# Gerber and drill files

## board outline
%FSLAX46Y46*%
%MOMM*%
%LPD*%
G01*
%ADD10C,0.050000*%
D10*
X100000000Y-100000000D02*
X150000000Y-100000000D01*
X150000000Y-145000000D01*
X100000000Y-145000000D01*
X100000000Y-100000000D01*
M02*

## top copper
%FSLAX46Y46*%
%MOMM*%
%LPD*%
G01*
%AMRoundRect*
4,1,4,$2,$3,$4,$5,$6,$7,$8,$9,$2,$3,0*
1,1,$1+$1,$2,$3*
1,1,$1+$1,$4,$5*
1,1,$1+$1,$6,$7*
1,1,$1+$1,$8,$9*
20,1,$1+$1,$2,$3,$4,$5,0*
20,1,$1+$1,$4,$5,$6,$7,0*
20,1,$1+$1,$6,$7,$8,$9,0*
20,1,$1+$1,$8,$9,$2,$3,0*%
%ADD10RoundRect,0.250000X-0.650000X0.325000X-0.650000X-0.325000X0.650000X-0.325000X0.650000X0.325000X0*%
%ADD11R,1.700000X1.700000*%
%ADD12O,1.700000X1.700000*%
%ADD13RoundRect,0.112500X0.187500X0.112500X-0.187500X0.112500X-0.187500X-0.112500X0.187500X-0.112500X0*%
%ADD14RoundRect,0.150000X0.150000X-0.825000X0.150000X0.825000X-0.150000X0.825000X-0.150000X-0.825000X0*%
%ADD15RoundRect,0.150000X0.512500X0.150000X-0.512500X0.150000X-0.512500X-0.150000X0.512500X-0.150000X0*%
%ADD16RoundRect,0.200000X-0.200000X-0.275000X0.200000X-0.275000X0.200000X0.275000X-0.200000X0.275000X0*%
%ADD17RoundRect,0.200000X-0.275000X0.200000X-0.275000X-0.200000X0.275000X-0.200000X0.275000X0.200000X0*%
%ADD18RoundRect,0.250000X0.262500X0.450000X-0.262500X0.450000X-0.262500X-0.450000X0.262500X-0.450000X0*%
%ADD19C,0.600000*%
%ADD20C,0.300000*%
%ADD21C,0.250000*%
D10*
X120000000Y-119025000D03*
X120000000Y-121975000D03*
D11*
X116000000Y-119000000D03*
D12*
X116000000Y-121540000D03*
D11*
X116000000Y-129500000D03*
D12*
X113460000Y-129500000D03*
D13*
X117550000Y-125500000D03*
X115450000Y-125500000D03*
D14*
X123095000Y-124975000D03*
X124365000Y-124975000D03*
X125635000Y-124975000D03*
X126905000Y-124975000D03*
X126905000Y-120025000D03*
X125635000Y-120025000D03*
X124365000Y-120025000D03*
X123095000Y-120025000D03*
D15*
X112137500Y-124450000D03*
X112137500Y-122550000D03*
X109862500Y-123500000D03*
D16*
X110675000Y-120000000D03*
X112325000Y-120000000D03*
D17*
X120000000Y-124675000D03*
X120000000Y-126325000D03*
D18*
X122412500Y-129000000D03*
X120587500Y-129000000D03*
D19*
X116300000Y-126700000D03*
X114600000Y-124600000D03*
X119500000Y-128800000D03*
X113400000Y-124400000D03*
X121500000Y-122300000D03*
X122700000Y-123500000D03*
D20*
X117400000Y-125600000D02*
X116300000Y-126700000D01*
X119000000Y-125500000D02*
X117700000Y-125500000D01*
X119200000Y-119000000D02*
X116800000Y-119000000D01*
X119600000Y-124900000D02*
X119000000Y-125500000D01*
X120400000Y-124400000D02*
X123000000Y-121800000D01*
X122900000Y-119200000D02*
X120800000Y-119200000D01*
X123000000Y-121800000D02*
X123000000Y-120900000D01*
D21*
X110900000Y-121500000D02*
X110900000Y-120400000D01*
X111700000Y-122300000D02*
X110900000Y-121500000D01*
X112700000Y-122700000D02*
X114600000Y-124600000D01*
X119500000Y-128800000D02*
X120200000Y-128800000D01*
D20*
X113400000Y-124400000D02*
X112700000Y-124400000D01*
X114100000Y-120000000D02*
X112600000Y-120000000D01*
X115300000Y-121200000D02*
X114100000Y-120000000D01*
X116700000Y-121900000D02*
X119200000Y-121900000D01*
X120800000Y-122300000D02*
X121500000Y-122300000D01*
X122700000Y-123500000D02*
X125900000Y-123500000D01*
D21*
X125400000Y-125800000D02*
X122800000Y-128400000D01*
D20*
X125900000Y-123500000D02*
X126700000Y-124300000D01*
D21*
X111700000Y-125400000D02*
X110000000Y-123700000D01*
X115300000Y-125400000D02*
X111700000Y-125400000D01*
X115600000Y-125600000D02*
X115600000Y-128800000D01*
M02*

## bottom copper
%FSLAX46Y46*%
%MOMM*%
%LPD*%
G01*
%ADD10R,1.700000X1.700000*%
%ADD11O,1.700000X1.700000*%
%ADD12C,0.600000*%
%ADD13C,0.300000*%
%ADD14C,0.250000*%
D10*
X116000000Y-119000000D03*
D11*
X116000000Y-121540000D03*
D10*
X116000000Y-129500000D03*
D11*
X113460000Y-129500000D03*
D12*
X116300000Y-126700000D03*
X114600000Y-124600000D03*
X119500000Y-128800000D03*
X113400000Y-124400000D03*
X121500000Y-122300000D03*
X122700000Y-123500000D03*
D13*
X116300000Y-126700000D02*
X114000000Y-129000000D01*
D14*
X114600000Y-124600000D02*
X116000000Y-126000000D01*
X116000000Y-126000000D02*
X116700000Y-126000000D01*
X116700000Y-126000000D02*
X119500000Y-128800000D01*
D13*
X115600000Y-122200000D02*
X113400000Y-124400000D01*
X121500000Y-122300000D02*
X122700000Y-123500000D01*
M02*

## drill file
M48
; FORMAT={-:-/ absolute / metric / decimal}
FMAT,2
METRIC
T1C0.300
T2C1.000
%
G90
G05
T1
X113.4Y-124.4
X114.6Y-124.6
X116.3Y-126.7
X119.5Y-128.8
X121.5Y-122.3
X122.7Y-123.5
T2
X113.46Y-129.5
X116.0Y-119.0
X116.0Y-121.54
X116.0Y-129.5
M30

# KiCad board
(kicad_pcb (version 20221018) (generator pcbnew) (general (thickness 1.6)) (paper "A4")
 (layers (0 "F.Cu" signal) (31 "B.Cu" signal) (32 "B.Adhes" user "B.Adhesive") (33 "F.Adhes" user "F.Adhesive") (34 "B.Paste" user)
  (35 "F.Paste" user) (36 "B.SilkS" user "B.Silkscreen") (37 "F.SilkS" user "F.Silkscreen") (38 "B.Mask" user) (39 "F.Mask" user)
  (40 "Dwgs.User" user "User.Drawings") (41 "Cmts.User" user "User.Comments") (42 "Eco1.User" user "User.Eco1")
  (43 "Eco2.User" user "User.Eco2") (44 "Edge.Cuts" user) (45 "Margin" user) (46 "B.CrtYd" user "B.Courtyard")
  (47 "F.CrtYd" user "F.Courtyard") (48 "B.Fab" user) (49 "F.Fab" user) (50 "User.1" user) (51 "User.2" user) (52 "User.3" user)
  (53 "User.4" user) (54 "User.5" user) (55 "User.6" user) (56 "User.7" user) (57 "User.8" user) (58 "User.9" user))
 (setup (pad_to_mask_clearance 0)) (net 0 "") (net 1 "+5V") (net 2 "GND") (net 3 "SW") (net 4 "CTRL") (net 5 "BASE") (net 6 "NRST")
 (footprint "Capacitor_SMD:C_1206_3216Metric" (layer "F.Cu") (at 120 120.5 -90)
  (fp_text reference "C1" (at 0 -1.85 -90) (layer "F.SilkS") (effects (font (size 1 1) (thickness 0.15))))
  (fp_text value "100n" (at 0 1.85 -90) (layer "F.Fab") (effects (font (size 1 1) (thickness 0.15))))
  (pad "1" smd roundrect (at -1.475 0 270) (size 1.15 1.8) (layers "F.Cu" "F.Paste" "F.Mask") (roundrect_rratio 0.217391) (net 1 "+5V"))
  (pad "2" smd roundrect (at 1.475 0 270) (size 1.15 1.8) (layers "F.Cu" "F.Paste" "F.Mask") (roundrect_rratio 0.217391) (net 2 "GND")))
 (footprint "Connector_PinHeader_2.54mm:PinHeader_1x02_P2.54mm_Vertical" (layer "F.Cu") (at 116 119)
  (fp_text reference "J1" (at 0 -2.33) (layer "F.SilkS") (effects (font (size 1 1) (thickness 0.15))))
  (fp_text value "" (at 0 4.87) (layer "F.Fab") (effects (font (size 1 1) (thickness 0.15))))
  (pad "1" thru_hole rect (at 0 0) (size 1.7 1.7) (drill 1) (layers "*.Cu" "*.Mask") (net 1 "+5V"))
  (pad "2" thru_hole oval (at 0 2.54) (size 1.7 1.7) (drill 1) (layers "*.Cu" "*.Mask") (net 2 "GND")))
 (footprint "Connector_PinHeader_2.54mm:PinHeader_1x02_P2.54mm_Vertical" (layer "F.Cu") (at 116 129.5 -90)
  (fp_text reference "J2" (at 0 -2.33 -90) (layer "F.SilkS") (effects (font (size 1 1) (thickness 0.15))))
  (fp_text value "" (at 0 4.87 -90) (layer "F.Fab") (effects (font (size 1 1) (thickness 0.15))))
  (pad "1" thru_hole rect (at 0 0 270) (size 1.7 1.7) (drill 1) (layers "*.Cu" "*.Mask") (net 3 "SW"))
  (pad "2" thru_hole oval (at 0 2.54 270) (size 1.7 1.7) (drill 1) (layers "*.Cu" "*.Mask") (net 1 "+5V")))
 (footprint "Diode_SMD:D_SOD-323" (layer "F.Cu") (at 116.5 125.5 180)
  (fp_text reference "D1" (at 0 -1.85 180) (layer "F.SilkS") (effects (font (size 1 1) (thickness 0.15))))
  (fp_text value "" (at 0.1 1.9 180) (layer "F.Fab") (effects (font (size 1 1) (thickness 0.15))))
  (pad "1" smd roundrect (at -1.05 0 180) (size 0.6 0.45) (layers "F.Cu" "F.Paste" "F.Mask") (roundrect_rratio 0.25) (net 1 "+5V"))
  (pad "2" smd roundrect (at 1.05 0 180) (size 0.6 0.45) (layers "F.Cu" "F.Paste" "F.Mask") (roundrect_rratio 0.25) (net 3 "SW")))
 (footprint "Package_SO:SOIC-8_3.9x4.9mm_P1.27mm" (layer "F.Cu") (at 125 122.5 90)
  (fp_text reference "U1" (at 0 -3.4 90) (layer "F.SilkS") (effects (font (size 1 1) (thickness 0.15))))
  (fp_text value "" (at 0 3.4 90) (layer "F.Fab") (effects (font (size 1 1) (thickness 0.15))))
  (pad "1" smd roundrect (at -2.475 -1.905 90) (size 1.95 0.6) (layers "F.Cu" "F.Paste" "F.Mask") (roundrect_rratio 0.25))
  (pad "2" smd roundrect (at -2.475 -0.635 90) (size 1.95 0.6) (layers "F.Cu" "F.Paste" "F.Mask") (roundrect_rratio 0.25))
  (pad "3" smd roundrect (at -2.475 0.635 90) (size 1.95 0.6) (layers "F.Cu" "F.Paste" "F.Mask") (roundrect_rratio 0.25) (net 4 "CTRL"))
  (pad "4" smd roundrect (at -2.475 1.905 90) (size 1.95 0.6) (layers "F.Cu" "F.Paste" "F.Mask") (roundrect_rratio 0.25) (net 2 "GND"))
  (pad "5" smd roundrect (at 2.475 1.905 90) (size 1.95 0.6) (layers "F.Cu" "F.Paste" "F.Mask") (roundrect_rratio 0.25))
  (pad "6" smd roundrect (at 2.475 0.635 90) (size 1.95 0.6) (layers "F.Cu" "F.Paste" "F.Mask") (roundrect_rratio 0.25))
  (pad "7" smd roundrect (at 2.475 -0.635 90) (size 1.95 0.6) (layers "F.Cu" "F.Paste" "F.Mask") (roundrect_rratio 0.25))
  (pad "8" smd roundrect (at 2.475 -1.905 90) (size 1.95 0.6) (layers "F.Cu" "F.Paste" "F.Mask") (roundrect_rratio 0.25) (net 1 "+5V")))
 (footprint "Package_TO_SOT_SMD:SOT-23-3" (layer "F.Cu") (at 111 123.5 180)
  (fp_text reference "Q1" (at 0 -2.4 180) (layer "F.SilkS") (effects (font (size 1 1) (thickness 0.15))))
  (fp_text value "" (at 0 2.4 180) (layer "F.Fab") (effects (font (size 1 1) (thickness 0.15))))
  (pad "1" smd roundrect (at -1.1375 -0.95 180) (size 1.325 0.6) (layers "F.Cu" "F.Paste" "F.Mask") (roundrect_rratio 0.25) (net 2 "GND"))
  (pad "2" smd roundrect (at -1.1375 0.95 180) (size 1.325 0.6) (layers "F.Cu" "F.Paste" "F.Mask") (roundrect_rratio 0.25) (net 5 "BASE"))
  (pad "3" smd roundrect (at 1.1375 0 180) (size 1.325 0.6) (layers "F.Cu" "F.Paste" "F.Mask") (roundrect_rratio 0.25) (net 3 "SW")))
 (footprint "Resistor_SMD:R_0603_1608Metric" (layer "F.Cu") (at 111.5 120)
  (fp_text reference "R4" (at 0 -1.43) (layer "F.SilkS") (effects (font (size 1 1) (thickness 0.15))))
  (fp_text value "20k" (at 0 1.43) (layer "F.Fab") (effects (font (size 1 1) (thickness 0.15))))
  (pad "1" smd roundrect (at -0.825 0) (size 0.8 0.95) (layers "F.Cu" "F.Paste" "F.Mask") (roundrect_rratio 0.25) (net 5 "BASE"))
  (pad "2" smd roundrect (at 0.825 0) (size 0.8 0.95) (layers "F.Cu" "F.Paste" "F.Mask") (roundrect_rratio 0.25) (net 2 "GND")))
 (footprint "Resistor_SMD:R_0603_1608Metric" (layer "F.Cu") (at 120 125.5 -90)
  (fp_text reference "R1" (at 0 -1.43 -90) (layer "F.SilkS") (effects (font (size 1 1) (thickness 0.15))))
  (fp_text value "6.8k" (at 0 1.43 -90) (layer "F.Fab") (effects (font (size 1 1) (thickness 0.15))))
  (pad "1" smd roundrect (at -0.825 0 270) (size 0.8 0.95) (layers "F.Cu" "F.Paste" "F.Mask") (roundrect_rratio 0.25) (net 1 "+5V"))
  (pad "2" smd roundrect (at 0.825 0 270) (size 0.8 0.95) (layers "F.Cu" "F.Paste" "F.Mask") (roundrect_rratio 0.25) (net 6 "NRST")))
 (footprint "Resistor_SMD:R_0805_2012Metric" (layer "F.Cu") (at 121.5 129 180)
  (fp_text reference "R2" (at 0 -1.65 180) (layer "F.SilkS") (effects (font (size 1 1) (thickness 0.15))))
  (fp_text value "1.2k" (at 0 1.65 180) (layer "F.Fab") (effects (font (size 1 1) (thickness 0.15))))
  (pad "1" smd roundrect (at -0.9125 0 180) (size 1.025 1.4) (layers "F.Cu" "F.Paste" "F.Mask") (roundrect_rratio 0.243902) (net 4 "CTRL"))
  (pad "2" smd roundrect (at 0.9125 0 180) (size 1.025 1.4) (layers "F.Cu" "F.Paste" "F.Mask") (roundrect_rratio 0.243902) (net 5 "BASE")))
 (gr_rect (start 100 100) (end 150 145) (stroke (width 0.05) (type default)) (fill none) (layer "Edge.Cuts"))
 (segment (start 117.4 125.6) (end 116.3 126.7) (width 0.3) (layer "F.Cu") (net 1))
 (segment (start 119 125.5) (end 117.7 125.5) (width 0.3) (layer "F.Cu") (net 1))
 (segment (start 119.2 119) (end 116.8 119) (width 0.3) (layer "F.Cu") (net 1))
 (segment (start 119.6 124.9) (end 119 125.5) (width 0.3) (layer "F.Cu") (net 1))
 (segment (start 120.4 124.4) (end 123 121.8) (width 0.3) (layer "F.Cu") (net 1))
 (segment (start 122.9 119.2) (end 120.8 119.2) (width 0.3) (layer "F.Cu") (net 1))
 (segment (start 123 121.8) (end 123 120.9) (width 0.3) (layer "F.Cu") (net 1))
 (via (at 116.3 126.7) (size 0.6) (drill 0.3) (layers "F.Cu" "B.Cu") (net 1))
 (segment (start 110.9 121.5) (end 110.9 120.4) (width 0.25) (layer "F.Cu") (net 5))
 (segment (start 111.7 122.3) (end 110.9 121.5) (width 0.25) (layer "F.Cu") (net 5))
 (segment (start 112.7 122.7) (end 114.6 124.6) (width 0.25) (layer "F.Cu") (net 5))
 (segment (start 116.3 126.7) (end 114 129) (width 0.3) (layer "B.Cu") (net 1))
 (segment (start 119.5 128.8) (end 120.2 128.8) (width 0.25) (layer "F.Cu") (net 5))
 (via (at 114.6 124.6) (size 0.6) (drill 0.3) (layers "F.Cu" "B.Cu") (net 5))
 (via (at 119.5 128.8) (size 0.6) (drill 0.3) (layers "F.Cu" "B.Cu") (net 5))
 (segment (start 113.4 124.4) (end 112.7 124.4) (width 0.3) (layer "F.Cu") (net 2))
 (segment (start 114.1 120) (end 112.6 120) (width 0.3) (layer "F.Cu") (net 2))
 (segment (start 114.6 124.6) (end 116 126) (width 0.25) (layer "B.Cu") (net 5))
 (segment (start 115.3 121.2) (end 114.1 120) (width 0.3) (layer "F.Cu") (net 2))
 (segment (start 116 126) (end 116.7 126) (width 0.25) (layer "B.Cu") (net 5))
 (segment (start 116.7 121.9) (end 119.2 121.9) (width 0.3) (layer "F.Cu") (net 2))
 (segment (start 116.7 126) (end 119.5 128.8) (width 0.25) (layer "B.Cu") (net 5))
 (segment (start 120.8 122.3) (end 121.5 122.3) (width 0.3) (layer "F.Cu") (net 2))
 (segment (start 122.7 123.5) (end 125.9 123.5) (width 0.3) (layer "F.Cu") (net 2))
 (segment (start 125.4 125.8) (end 122.8 128.4) (width 0.25) (layer "F.Cu") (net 4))
 (segment (start 125.9 123.5) (end 126.7 124.3) (width 0.3) (layer "F.Cu") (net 2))
 (via (at 113.4 124.4) (size 0.6) (drill 0.3) (layers "F.Cu" "B.Cu") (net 2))
 (via (at 121.5 122.3) (size 0.6) (drill 0.3) (layers "F.Cu" "B.Cu") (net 2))
 (via (at 122.7 123.5) (size 0.6) (drill 0.3) (layers "F.Cu" "B.Cu") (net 2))
 (segment (start 111.7 125.4) (end 110 123.7) (width 0.25) (layer "F.Cu") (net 3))
 (segment (start 115.3 125.4) (end 111.7 125.4) (width 0.25) (layer "F.Cu") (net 3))
 (segment (start 115.6 122.2) (end 113.4 124.4) (width 0.3) (layer "B.Cu") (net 2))
 (segment (start 115.6 125.6) (end 115.6 128.8) (width 0.25) (layer "F.Cu") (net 3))
 (segment (start 121.5 122.3) (end 122.7 123.5) (width 0.3) (layer "B.Cu") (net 2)))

